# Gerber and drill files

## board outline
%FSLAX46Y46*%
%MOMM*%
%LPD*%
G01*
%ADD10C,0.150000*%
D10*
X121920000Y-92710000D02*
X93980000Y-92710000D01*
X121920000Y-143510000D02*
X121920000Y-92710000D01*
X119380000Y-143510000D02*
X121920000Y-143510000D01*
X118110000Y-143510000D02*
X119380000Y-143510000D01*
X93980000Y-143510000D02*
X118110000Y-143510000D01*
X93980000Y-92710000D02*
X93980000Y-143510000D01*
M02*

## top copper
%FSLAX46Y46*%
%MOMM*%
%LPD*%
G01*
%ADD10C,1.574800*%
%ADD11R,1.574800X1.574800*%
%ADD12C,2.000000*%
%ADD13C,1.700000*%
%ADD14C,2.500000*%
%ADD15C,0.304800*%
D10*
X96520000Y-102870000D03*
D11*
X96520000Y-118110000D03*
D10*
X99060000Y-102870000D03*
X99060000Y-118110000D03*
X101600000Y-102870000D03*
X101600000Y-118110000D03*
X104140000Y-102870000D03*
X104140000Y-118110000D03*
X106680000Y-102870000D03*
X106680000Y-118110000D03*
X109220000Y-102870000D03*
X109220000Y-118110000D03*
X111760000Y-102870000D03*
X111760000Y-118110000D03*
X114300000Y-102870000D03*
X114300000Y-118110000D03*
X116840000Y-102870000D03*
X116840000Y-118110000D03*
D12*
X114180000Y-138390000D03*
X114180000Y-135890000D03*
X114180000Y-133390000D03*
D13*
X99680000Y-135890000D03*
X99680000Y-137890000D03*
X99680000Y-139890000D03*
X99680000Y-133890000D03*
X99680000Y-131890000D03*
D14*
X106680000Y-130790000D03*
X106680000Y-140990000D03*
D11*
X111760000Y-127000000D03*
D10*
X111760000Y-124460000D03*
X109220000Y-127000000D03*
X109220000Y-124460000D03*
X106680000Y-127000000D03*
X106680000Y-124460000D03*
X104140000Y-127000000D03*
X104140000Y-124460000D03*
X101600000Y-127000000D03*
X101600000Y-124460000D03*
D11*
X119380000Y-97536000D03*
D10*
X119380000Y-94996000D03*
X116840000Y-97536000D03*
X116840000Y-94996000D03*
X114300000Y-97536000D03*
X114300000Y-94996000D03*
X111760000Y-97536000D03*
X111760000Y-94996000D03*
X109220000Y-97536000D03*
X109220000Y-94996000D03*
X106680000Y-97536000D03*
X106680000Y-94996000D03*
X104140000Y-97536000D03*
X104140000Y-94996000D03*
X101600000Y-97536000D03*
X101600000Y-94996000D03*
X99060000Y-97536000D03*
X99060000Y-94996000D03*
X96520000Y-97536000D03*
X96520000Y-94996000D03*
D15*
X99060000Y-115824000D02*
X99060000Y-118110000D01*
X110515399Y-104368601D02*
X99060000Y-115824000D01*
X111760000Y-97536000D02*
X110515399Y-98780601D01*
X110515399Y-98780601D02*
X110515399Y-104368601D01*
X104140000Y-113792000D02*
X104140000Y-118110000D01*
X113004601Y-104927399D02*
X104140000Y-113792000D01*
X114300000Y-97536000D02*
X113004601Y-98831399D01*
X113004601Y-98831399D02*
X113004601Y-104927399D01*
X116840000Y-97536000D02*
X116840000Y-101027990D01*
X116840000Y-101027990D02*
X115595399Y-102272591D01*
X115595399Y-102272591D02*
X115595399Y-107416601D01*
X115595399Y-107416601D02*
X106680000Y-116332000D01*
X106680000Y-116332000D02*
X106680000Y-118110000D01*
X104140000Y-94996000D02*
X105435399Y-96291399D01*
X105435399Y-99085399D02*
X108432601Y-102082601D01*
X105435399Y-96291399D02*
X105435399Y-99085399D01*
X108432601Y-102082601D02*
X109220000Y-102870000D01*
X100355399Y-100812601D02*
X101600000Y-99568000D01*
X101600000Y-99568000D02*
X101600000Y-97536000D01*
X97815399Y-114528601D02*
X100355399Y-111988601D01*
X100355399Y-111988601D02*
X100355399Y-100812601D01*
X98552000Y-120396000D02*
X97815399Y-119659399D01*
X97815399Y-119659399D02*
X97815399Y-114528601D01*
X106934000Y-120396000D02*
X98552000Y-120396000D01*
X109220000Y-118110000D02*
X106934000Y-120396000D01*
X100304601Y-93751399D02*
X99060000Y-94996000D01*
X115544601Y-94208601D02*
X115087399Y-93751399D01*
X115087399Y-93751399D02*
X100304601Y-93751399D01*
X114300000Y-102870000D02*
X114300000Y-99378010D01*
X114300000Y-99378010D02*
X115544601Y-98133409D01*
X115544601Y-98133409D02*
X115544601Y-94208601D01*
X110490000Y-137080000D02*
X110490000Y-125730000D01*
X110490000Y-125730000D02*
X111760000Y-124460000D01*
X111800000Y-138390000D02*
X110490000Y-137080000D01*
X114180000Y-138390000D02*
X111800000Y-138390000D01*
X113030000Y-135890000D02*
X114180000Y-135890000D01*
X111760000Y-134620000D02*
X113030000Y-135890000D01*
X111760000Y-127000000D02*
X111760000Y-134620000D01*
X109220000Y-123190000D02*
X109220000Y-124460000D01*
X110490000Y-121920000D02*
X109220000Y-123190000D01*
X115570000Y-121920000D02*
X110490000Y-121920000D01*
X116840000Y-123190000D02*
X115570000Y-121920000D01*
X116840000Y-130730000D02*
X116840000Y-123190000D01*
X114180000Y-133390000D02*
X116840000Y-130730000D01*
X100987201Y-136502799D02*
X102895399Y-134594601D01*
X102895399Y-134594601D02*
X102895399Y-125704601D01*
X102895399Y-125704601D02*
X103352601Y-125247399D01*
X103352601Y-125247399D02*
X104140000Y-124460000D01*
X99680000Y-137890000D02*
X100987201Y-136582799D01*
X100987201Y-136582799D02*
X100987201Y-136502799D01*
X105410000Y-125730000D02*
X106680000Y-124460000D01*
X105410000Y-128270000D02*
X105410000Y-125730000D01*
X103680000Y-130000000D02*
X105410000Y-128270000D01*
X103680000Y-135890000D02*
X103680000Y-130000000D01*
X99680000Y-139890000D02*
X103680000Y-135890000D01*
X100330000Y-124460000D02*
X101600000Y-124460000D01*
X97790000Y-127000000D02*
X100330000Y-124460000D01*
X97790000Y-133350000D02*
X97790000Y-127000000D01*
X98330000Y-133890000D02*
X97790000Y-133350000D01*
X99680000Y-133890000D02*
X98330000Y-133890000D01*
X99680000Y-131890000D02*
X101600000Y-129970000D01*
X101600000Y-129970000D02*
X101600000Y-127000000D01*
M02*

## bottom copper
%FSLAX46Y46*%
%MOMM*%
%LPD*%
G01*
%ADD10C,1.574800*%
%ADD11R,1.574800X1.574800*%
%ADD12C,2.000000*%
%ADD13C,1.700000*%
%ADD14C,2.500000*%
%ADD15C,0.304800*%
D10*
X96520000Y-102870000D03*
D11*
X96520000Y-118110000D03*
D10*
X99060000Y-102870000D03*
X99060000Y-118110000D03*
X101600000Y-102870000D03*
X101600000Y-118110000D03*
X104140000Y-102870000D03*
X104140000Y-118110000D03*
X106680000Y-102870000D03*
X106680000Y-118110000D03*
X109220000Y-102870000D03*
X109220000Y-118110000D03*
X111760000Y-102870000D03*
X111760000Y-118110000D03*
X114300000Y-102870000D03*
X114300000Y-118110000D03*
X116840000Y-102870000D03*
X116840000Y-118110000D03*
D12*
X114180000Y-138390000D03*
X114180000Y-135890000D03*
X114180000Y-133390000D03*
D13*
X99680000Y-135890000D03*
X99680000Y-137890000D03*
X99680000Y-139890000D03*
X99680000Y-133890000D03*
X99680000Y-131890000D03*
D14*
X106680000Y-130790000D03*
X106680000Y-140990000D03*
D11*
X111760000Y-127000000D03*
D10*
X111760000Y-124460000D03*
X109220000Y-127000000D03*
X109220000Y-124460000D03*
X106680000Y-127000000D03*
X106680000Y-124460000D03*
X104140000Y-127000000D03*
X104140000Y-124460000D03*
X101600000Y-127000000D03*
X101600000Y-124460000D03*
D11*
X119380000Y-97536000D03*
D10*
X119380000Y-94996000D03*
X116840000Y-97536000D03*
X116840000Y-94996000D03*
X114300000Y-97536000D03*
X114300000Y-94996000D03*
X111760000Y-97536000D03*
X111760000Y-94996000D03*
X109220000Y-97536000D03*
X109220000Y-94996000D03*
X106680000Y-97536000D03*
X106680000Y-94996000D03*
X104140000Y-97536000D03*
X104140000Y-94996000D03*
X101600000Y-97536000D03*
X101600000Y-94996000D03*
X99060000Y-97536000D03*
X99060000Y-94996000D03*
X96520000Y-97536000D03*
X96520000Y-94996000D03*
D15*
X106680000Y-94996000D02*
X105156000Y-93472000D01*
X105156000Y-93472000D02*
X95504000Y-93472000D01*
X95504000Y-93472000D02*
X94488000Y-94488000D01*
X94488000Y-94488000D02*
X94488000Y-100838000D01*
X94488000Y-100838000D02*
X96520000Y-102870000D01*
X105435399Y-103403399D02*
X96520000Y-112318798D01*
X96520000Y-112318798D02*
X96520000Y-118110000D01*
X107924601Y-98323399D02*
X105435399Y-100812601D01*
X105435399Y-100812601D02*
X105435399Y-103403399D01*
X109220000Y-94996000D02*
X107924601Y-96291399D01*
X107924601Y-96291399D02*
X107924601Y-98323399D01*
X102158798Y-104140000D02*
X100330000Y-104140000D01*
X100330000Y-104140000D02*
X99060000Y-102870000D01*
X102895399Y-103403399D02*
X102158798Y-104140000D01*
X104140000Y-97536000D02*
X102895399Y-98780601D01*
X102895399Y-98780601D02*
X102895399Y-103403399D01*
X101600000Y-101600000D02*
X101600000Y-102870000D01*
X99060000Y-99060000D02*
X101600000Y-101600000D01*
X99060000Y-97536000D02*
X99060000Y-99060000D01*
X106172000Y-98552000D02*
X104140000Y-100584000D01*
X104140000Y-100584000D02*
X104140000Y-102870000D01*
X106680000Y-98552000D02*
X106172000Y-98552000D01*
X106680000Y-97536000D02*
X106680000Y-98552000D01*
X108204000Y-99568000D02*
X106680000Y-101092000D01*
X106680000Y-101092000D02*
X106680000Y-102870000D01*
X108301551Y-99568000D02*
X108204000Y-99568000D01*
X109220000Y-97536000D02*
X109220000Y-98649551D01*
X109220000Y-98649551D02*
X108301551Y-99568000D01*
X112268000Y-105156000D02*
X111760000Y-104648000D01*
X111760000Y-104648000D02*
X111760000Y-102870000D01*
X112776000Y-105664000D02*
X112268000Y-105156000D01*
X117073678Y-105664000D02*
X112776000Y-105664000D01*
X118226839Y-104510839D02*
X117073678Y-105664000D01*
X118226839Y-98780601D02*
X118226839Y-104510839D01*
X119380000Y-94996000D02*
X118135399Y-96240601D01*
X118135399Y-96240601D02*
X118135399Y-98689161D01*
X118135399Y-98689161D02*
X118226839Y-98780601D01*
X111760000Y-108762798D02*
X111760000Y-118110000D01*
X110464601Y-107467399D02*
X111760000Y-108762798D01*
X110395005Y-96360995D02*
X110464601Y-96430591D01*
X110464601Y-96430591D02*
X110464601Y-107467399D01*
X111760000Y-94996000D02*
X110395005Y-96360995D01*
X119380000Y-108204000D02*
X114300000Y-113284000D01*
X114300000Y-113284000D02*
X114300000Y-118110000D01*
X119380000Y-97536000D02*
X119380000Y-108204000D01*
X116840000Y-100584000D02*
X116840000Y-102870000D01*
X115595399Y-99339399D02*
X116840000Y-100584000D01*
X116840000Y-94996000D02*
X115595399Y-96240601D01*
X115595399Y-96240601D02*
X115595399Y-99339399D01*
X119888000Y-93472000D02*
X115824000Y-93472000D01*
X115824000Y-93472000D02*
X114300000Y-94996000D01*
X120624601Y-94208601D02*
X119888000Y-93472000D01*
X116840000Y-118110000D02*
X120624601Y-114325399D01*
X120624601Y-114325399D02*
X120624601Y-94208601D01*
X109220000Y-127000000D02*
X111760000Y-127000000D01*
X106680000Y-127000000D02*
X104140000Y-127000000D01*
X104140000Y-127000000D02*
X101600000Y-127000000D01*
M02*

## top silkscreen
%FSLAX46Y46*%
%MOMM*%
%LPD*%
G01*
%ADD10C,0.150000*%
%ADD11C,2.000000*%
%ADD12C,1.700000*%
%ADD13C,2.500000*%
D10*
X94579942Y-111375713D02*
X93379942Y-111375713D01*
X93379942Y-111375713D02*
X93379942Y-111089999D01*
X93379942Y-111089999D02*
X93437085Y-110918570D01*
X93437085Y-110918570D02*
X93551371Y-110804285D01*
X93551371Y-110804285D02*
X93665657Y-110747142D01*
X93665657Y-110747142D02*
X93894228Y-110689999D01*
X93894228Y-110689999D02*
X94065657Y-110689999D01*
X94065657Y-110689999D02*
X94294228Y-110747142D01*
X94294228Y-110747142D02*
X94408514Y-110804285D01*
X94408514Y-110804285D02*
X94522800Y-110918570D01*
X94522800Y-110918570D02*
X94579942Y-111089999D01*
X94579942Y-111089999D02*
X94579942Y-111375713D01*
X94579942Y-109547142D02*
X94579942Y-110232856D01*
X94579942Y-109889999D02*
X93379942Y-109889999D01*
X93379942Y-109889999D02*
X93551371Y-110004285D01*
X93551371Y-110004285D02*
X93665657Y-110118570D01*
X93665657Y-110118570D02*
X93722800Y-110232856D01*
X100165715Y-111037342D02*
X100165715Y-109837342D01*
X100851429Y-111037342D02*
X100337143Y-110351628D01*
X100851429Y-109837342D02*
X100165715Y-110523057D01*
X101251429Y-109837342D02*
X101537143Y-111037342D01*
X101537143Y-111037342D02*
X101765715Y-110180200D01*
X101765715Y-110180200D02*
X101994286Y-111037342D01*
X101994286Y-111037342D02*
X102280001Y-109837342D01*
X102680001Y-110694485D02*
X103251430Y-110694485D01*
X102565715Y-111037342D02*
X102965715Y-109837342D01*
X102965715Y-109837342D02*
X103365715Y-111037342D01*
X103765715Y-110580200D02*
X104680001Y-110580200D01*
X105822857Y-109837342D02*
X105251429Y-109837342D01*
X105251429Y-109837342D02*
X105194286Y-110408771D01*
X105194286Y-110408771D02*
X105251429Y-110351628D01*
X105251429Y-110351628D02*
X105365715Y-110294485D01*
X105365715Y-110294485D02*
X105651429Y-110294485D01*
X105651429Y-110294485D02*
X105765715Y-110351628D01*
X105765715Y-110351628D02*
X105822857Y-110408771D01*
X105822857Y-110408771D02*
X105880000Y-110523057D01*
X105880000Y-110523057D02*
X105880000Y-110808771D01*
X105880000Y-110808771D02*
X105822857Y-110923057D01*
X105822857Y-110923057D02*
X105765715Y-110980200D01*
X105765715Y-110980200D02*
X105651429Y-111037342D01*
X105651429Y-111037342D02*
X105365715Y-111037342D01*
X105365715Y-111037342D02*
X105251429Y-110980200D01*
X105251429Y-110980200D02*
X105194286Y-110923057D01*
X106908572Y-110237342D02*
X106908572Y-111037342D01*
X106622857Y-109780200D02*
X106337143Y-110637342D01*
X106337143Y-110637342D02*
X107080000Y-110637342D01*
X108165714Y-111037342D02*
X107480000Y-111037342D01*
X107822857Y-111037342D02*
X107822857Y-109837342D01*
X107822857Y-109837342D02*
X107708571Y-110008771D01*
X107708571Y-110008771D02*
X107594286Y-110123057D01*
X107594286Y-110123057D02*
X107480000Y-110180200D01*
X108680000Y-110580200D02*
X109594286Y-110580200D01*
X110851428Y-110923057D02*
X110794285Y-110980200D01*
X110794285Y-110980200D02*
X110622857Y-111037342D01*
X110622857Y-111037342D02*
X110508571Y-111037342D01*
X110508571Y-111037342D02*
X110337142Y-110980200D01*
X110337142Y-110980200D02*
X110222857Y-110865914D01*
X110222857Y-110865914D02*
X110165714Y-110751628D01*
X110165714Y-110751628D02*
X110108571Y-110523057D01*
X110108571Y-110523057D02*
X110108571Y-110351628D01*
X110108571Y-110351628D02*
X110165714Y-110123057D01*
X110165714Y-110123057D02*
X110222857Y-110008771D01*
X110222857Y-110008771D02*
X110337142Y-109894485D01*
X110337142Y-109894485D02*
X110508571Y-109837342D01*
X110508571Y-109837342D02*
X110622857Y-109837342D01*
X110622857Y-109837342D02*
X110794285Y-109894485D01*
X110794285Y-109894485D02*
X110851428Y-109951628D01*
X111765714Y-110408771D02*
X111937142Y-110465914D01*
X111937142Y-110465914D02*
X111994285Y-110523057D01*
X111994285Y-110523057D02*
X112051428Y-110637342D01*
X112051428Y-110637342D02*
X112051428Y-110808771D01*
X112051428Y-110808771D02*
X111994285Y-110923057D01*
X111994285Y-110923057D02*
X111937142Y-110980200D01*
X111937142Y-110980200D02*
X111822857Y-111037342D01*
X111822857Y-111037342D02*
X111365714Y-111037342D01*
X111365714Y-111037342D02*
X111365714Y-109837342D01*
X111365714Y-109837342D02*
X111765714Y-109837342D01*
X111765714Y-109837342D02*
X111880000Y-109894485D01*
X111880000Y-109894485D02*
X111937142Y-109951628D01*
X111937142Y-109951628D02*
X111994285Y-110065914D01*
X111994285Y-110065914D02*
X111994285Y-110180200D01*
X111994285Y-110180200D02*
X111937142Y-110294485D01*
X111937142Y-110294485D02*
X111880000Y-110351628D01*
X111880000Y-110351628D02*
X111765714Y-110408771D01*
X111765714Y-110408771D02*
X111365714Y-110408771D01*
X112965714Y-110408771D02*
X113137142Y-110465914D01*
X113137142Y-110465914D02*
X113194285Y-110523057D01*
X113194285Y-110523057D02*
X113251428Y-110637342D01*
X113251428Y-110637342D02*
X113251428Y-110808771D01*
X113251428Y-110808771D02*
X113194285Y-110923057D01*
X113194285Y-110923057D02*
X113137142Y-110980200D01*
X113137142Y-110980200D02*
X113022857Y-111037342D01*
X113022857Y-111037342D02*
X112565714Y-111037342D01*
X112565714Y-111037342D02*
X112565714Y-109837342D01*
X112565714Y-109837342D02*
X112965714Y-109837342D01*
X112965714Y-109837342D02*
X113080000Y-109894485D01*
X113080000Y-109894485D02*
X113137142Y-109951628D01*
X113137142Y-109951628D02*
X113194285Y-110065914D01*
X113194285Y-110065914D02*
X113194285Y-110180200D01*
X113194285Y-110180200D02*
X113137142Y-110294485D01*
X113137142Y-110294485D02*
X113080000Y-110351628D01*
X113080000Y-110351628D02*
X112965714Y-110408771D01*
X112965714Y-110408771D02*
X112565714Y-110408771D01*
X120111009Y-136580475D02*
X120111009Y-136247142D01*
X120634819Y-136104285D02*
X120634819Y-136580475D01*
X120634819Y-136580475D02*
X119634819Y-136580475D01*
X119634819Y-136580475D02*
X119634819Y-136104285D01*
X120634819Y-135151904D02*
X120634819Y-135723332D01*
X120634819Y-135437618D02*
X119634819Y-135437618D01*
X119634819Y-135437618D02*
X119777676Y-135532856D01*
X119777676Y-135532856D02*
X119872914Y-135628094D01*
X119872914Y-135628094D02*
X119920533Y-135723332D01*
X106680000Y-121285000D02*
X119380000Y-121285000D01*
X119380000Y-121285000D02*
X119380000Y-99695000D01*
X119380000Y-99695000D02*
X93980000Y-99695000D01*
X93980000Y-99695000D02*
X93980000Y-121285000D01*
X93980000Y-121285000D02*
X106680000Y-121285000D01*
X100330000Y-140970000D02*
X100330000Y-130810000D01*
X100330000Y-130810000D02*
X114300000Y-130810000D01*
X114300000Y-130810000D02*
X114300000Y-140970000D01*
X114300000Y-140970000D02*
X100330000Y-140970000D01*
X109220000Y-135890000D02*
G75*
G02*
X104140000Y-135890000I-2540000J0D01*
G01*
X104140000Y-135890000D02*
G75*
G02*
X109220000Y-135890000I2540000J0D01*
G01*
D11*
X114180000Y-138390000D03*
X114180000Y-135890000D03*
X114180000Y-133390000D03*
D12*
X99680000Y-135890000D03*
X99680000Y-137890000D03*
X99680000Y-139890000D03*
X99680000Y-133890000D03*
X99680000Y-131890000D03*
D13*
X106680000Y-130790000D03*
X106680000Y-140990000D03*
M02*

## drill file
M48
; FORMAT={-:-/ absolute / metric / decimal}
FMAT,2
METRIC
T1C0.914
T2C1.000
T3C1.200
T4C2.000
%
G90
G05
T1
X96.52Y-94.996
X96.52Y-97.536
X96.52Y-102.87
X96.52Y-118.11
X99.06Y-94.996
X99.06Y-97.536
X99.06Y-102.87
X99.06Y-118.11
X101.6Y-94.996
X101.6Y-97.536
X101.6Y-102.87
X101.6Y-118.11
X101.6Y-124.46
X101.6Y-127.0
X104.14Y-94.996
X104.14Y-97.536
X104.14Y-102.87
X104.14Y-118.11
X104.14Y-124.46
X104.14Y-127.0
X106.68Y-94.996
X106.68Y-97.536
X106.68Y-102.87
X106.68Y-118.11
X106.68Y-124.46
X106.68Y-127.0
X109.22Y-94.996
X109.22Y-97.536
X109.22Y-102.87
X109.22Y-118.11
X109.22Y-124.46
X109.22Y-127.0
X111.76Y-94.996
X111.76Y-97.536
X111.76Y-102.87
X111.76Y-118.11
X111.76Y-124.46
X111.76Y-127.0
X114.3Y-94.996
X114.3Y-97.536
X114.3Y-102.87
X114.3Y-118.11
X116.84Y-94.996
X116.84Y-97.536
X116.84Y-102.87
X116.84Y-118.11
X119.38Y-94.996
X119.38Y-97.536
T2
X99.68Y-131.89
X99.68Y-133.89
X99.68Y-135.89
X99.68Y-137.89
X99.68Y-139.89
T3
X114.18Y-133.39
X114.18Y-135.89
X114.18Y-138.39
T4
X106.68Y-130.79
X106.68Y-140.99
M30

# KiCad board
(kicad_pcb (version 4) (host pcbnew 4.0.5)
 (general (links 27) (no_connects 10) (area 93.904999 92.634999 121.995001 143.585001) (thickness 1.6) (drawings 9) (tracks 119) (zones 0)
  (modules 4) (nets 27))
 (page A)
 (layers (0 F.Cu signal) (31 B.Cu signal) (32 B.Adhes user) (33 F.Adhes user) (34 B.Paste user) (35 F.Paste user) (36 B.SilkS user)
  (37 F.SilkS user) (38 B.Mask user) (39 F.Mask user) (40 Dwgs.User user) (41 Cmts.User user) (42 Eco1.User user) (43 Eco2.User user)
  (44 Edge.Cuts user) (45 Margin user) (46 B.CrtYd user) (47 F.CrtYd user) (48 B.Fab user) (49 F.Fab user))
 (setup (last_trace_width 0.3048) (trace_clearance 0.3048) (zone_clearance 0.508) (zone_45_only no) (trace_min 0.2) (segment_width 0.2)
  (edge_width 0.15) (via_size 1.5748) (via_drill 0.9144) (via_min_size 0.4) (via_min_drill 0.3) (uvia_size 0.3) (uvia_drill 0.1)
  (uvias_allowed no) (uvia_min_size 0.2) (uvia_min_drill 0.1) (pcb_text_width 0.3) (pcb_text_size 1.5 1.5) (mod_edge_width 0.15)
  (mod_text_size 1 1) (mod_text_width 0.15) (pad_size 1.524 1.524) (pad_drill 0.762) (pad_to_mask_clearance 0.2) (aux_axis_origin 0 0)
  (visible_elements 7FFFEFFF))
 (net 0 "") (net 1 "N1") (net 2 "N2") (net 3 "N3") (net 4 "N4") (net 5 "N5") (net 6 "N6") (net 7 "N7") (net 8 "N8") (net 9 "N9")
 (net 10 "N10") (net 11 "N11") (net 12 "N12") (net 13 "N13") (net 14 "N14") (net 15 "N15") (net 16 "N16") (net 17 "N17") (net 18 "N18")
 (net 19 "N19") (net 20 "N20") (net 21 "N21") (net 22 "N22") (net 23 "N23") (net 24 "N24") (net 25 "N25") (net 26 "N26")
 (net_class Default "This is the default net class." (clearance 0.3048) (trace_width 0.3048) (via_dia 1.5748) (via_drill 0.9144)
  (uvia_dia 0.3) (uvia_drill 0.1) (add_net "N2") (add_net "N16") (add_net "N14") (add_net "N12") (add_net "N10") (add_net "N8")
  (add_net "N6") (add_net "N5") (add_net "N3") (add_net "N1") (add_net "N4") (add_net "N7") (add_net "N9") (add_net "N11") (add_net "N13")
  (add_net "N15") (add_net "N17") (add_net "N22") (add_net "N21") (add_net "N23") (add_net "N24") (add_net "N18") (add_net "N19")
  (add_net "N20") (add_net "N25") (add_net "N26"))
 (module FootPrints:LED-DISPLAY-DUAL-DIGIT (layer F.Cu) (at 106.68 110.49)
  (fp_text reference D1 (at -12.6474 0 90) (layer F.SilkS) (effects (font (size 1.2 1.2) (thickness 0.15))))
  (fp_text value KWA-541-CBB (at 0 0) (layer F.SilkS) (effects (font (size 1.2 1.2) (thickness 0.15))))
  (fp_line (start 0 10.795) (end 12.7 10.795) (layer F.SilkS) (width 0.15))
  (fp_line (start 12.7 10.795) (end 12.7 -10.795) (layer F.SilkS) (width 0.15))
  (fp_line (start 12.7 -10.795) (end -12.7 -10.795) (layer F.SilkS) (width 0.15))
  (fp_line (start -12.7 -10.795) (end -12.7 10.795) (layer F.SilkS) (width 0.15))
  (fp_line (start -12.7 10.795) (end 0 10.795) (layer F.SilkS) (width 0.15))
  (pad 18 thru_hole circle (at -10.16 -7.62) (size 1.5748 1.5748) (drill 0.9144) (layers *.Cu *.Mask) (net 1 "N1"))
  (pad 1 thru_hole rect (at -10.16 7.62) (size 1.5748 1.5748) (drill 0.9144) (layers *.Cu *.Mask) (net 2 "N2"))
  (pad 17 thru_hole circle (at -7.62 -7.62) (size 1.5748 1.5748) (drill 0.9144) (layers *.Cu *.Mask) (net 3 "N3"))
  (pad 2 thru_hole circle (at -7.62 7.62) (size 1.5748 1.5748) (drill 0.9144) (layers *.Cu *.Mask) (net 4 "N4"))
  (pad 16 thru_hole circle (at -5.08 -7.62) (size 1.5748 1.5748) (drill 0.9144) (layers *.Cu *.Mask) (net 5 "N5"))
  (pad 3 thru_hole circle (at -5.08 7.62) (size 1.5748 1.5748) (drill 0.9144) (layers *.Cu *.Mask))
  (pad 15 thru_hole circle (at -2.54 -7.62) (size 1.5748 1.5748) (drill 0.9144) (layers *.Cu *.Mask) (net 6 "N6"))
  (pad 4 thru_hole circle (at -2.54 7.62) (size 1.5748 1.5748) (drill 0.9144) (layers *.Cu *.Mask) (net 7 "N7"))
  (pad 14 thru_hole circle (at 0 -7.62) (size 1.5748 1.5748) (drill 0.9144) (layers *.Cu *.Mask) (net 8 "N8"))
  (pad 5 thru_hole circle (at 0 7.62) (size 1.5748 1.5748) (drill 0.9144) (layers *.Cu *.Mask) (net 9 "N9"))
  (pad 13 thru_hole circle (at 2.54 -7.62) (size 1.5748 1.5748) (drill 0.9144) (layers *.Cu *.Mask) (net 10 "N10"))
  (pad 6 thru_hole circle (at 2.54 7.62) (size 1.5748 1.5748) (drill 0.9144) (layers *.Cu *.Mask) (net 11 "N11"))
  (pad 12 thru_hole circle (at 5.08 -7.62) (size 1.5748 1.5748) (drill 0.9144) (layers *.Cu *.Mask) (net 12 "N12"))
  (pad 7 thru_hole circle (at 5.08 7.62) (size 1.5748 1.5748) (drill 0.9144) (layers *.Cu *.Mask) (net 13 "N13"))
  (pad 11 thru_hole circle (at 7.62 -7.62) (size 1.5748 1.5748) (drill 0.9144) (layers *.Cu *.Mask) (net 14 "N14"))
  (pad 8 thru_hole circle (at 7.62 7.62) (size 1.5748 1.5748) (drill 0.9144) (layers *.Cu *.Mask) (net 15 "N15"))
  (pad 10 thru_hole circle (at 10.16 -7.62) (size 1.5748 1.5748) (drill 0.9144) (layers *.Cu *.Mask) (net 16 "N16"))
  (pad 9 thru_hole circle (at 10.16 7.62) (size 1.5748 1.5748) (drill 0.9144) (layers *.Cu *.Mask) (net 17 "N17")))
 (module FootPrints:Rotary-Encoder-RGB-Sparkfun (layer F.Cu) (at 106.68 135.89 90)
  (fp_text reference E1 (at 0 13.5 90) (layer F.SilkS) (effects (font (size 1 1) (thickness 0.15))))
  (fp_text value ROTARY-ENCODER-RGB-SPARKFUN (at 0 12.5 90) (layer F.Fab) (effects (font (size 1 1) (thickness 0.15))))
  (fp_line (start -5.08 -6.35) (end 5.08 -6.35) (layer F.SilkS) (width 0.15))
  (fp_line (start 5.08 -6.35) (end 5.08 7.62) (layer F.SilkS) (width 0.15))
  (fp_line (start 5.08 7.62) (end -5.08 7.62) (layer F.SilkS) (width 0.15))
  (fp_line (start -5.08 7.62) (end -5.08 -6.35) (layer F.SilkS) (width 0.15))
  (fp_circle (center 0 0) (end 2.54 0) (layer F.SilkS) (width 0.15))
  (pad 6 thru_hole circle (at -2.5 7.5 90) (size 2 2) (drill 1.2) (layers *.Cu *.Mask F.SilkS) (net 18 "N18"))
  (pad 7 thru_hole circle (at 0 7.5 90) (size 2 2) (drill 1.2) (layers *.Cu *.Mask F.SilkS) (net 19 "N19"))
  (pad 8 thru_hole circle (at 2.5 7.5 90) (size 2 2) (drill 1.2) (layers *.Cu *.Mask F.SilkS) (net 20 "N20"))
  (pad 3 thru_hole circle (at 0 -7 90) (size 1.7 1.7) (drill 1) (layers *.Cu *.Mask F.SilkS))
  (pad 2 thru_hole circle (at -2 -7 90) (size 1.7 1.7) (drill 1) (layers *.Cu *.Mask F.SilkS) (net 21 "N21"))
  (pad 1 thru_hole circle (at -4 -7 90) (size 1.7 1.7) (drill 1) (layers *.Cu *.Mask F.SilkS) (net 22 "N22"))
  (pad 4 thru_hole circle (at 2 -7 90) (size 1.7 1.7) (drill 1) (layers *.Cu *.Mask F.SilkS) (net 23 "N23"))
  (pad 5 thru_hole circle (at 4 -7 90) (size 1.7 1.7) (drill 1) (layers *.Cu *.Mask F.SilkS) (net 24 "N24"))
  (pad "" thru_hole circle (at 5.1 0 90) (size 2.5 2.5) (drill 2) (layers *.Cu *.Mask F.SilkS))
  (pad "" thru_hole circle (at -5.1 0 90) (size 2.5 2.5) (drill 2) (layers *.Cu *.Mask F.SilkS)))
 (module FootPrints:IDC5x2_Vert (layer B.Cu) (at 106.68 125.73)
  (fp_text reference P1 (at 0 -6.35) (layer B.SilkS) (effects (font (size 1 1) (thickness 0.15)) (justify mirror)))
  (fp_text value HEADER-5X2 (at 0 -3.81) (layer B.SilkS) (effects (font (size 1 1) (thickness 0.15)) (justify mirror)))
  (pad 1 thru_hole rect (at 5.08 1.27) (size 1.5748 1.5748) (drill 0.9144) (layers *.Cu *.Mask B.SilkS) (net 19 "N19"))
  (pad 2 thru_hole circle (at 5.08 -1.27) (size 1.5748 1.5748) (drill 0.9144) (layers *.Cu *.Mask B.SilkS) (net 18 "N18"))
  (pad 3 thru_hole circle (at 2.54 1.27) (size 1.5748 1.5748) (drill 0.9144) (layers *.Cu *.Mask B.SilkS) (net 19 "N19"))
  (pad 4 thru_hole circle (at 2.54 -1.27) (size 1.5748 1.5748) (drill 0.9144) (layers *.Cu *.Mask B.SilkS) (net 20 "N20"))
  (pad 5 thru_hole circle (at 0 1.27) (size 1.5748 1.5748) (drill 0.9144) (layers *.Cu *.Mask B.SilkS) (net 24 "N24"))
  (pad 6 thru_hole circle (at 0 -1.27) (size 1.5748 1.5748) (drill 0.9144) (layers *.Cu *.Mask B.SilkS) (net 22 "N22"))
  (pad 7 thru_hole circle (at -2.54 1.27) (size 1.5748 1.5748) (drill 0.9144) (layers *.Cu *.Mask B.SilkS) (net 24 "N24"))
  (pad 8 thru_hole circle (at -2.54 -1.27) (size 1.5748 1.5748) (drill 0.9144) (layers *.Cu *.Mask B.SilkS) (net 21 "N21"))
  (pad 9 thru_hole circle (at -5.08 1.27) (size 1.5748 1.5748) (drill 0.9144) (layers *.Cu *.Mask B.SilkS) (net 24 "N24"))
  (pad 10 thru_hole circle (at -5.08 -1.27) (size 1.5748 1.5748) (drill 0.9144) (layers *.Cu *.Mask B.SilkS) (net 23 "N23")))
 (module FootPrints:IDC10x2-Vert (layer B.Cu) (at 111.76 102.616 180)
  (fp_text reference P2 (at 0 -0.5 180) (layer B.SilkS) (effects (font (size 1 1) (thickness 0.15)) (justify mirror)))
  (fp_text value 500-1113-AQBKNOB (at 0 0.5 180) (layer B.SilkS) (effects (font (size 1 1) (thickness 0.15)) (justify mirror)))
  (pad 1 thru_hole rect (at -7.62 5.08 180) (size 1.5748 1.5748) (drill 0.9144) (layers *.Cu *.Mask) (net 15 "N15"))
  (pad 2 thru_hole circle (at -7.62 7.62 180) (size 1.5748 1.5748) (drill 0.9144) (layers *.Cu *.Mask) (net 12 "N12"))
  (pad 3 thru_hole circle (at -5.08 5.08 180) (size 1.5748 1.5748) (drill 0.9144) (layers *.Cu *.Mask) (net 9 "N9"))
  (pad 4 thru_hole circle (at -5.08 7.62 180) (size 1.5748 1.5748) (drill 0.9144) (layers *.Cu *.Mask) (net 16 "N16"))
  (pad 5 thru_hole circle (at -2.54 5.08 180) (size 1.5748 1.5748) (drill 0.9144) (layers *.Cu *.Mask) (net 7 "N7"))
  (pad 6 thru_hole circle (at -2.54 7.62 180) (size 1.5748 1.5748) (drill 0.9144) (layers *.Cu *.Mask) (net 17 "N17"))
  (pad 7 thru_hole circle (at 0 5.08 180) (size 1.5748 1.5748) (drill 0.9144) (layers *.Cu *.Mask) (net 4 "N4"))
  (pad 8 thru_hole circle (at 0 7.62 180) (size 1.5748 1.5748) (drill 0.9144) (layers *.Cu *.Mask) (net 13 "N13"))
  (pad 9 thru_hole circle (at 2.54 5.08 180) (size 1.5748 1.5748) (drill 0.9144) (layers *.Cu *.Mask) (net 8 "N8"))
  (pad 10 thru_hole circle (at 2.54 7.62 180) (size 1.5748 1.5748) (drill 0.9144) (layers *.Cu *.Mask) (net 2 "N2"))
  (pad 11 thru_hole circle (at 5.08 5.08 180) (size 1.5748 1.5748) (drill 0.9144) (layers *.Cu *.Mask) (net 6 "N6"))
  (pad 12 thru_hole circle (at 5.08 7.62 180) (size 1.5748 1.5748) (drill 0.9144) (layers *.Cu *.Mask) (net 1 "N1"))
  (pad 13 thru_hole circle (at 7.62 5.08 180) (size 1.5748 1.5748) (drill 0.9144) (layers *.Cu *.Mask) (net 3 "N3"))
  (pad 14 thru_hole circle (at 7.62 7.62 180) (size 1.5748 1.5748) (drill 0.9144) (layers *.Cu *.Mask) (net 10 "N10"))
  (pad 15 thru_hole circle (at 10.16 5.08 180) (size 1.5748 1.5748) (drill 0.9144) (layers *.Cu *.Mask) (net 11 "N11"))
  (pad 16 thru_hole circle (at 10.16 7.62 180) (size 1.5748 1.5748) (drill 0.9144) (layers *.Cu *.Mask))
  (pad 17 thru_hole circle (at 12.7 5.08 180) (size 1.5748 1.5748) (drill 0.9144) (layers *.Cu *.Mask) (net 5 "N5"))
  (pad 18 thru_hole circle (at 12.7 7.62 180) (size 1.5748 1.5748) (drill 0.9144) (layers *.Cu *.Mask) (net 14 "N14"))
  (pad 19 thru_hole circle (at 15.24 5.08 180) (size 1.5748 1.5748) (drill 0.9144) (layers *.Cu *.Mask) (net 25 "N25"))
  (pad 20 thru_hole circle (at 15.24 7.62 180) (size 1.5748 1.5748) (drill 0.9144) (layers *.Cu *.Mask) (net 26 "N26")))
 (gr_line (start 121.92 92.71) (end 93.98 92.71) (angle 90) (layer Edge.Cuts) (width 0.15))
 (gr_line (start 121.92 143.51) (end 121.92 92.71) (angle 90) (layer Edge.Cuts) (width 0.15))
 (gr_line (start 119.38 143.51) (end 121.92 143.51) (angle 90) (layer Edge.Cuts) (width 0.15))
 (gr_line (start 118.11 143.51) (end 119.38 143.51) (angle 90) (layer Edge.Cuts) (width 0.15))
 (gr_line (start 93.98 143.51) (end 118.11 143.51) (angle 90) (layer Edge.Cuts) (width 0.15))
 (gr_line (start 93.98 92.71) (end 93.98 143.51) (angle 90) (layer Edge.Cuts) (width 0.15))
 (segment (start 106.68 94.996) (end 105.156 93.472) (width 0.3048) (layer B.Cu) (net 1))
 (segment (start 105.156 93.472) (end 95.504 93.472) (width 0.3048) (layer B.Cu) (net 1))
 (segment (start 95.504 93.472) (end 94.488 94.488) (width 0.3048) (layer B.Cu) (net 1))
 (segment (start 94.488 94.488) (end 94.488 100.838) (width 0.3048) (layer B.Cu) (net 1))
 (segment (start 94.488 100.838) (end 96.52 102.87) (width 0.3048) (layer B.Cu) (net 1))
 (segment (start 105.435399 103.403399) (end 96.52 112.318798) (width 0.3048) (layer B.Cu) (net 2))
 (segment (start 96.52 112.318798) (end 96.52 118.11) (width 0.3048) (layer B.Cu) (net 2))
 (segment (start 107.924601 98.323399) (end 105.435399 100.812601) (width 0.3048) (layer B.Cu) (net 2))
 (segment (start 105.435399 100.812601) (end 105.435399 103.403399) (width 0.3048) (layer B.Cu) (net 2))
 (segment (start 109.22 94.996) (end 107.924601 96.291399) (width 0.3048) (layer B.Cu) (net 2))
 (segment (start 107.924601 96.291399) (end 107.924601 98.323399) (width 0.3048) (layer B.Cu) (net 2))
 (segment (start 102.158798 104.14) (end 100.33 104.14) (width 0.3048) (layer B.Cu) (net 3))
 (segment (start 100.33 104.14) (end 99.06 102.87) (width 0.3048) (layer B.Cu) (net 3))
 (segment (start 102.895399 103.403399) (end 102.158798 104.14) (width 0.3048) (layer B.Cu) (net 3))
 (segment (start 104.14 97.536) (end 102.895399 98.780601) (width 0.3048) (layer B.Cu) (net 3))
 (segment (start 102.895399 98.780601) (end 102.895399 103.403399) (width 0.3048) (layer B.Cu) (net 3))
 (segment (start 99.06 115.824) (end 99.06 118.11) (width 0.3048) (layer F.Cu) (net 4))
 (segment (start 110.515399 104.368601) (end 99.06 115.824) (width 0.3048) (layer F.Cu) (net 4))
 (segment (start 111.76 97.536) (end 110.515399 98.780601) (width 0.3048) (layer F.Cu) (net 4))
 (segment (start 110.515399 98.780601) (end 110.515399 104.368601) (width 0.3048) (layer F.Cu) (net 4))
 (segment (start 101.6 101.6) (end 101.6 102.87) (width 0.3048) (layer B.Cu) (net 5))
 (segment (start 99.06 99.06) (end 101.6 101.6) (width 0.3048) (layer B.Cu) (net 5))
 (segment (start 99.06 97.536) (end 99.06 99.06) (width 0.3048) (layer B.Cu) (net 5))
 (segment (start 106.172 98.552) (end 104.14 100.584) (width 0.3048) (layer B.Cu) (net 6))
 (segment (start 104.14 100.584) (end 104.14 102.87) (width 0.3048) (layer B.Cu) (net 6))
 (segment (start 106.68 98.552) (end 106.172 98.552) (width 0.3048) (layer B.Cu) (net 6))
 (segment (start 106.68 97.536) (end 106.68 98.552) (width 0.3048) (layer B.Cu) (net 6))
 (segment (start 104.14 113.792) (end 104.14 118.11) (width 0.3048) (layer F.Cu) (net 7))
 (segment (start 113.004601 104.927399) (end 104.14 113.792) (width 0.3048) (layer F.Cu) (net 7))
 (segment (start 114.3 97.536) (end 113.004601 98.831399) (width 0.3048) (layer F.Cu) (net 7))
 (segment (start 113.004601 98.831399) (end 113.004601 104.927399) (width 0.3048) (layer F.Cu) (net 7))
 (segment (start 108.204 99.568) (end 106.68 101.092) (width 0.3048) (layer B.Cu) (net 8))
 (segment (start 106.68 101.092) (end 106.68 102.87) (width 0.3048) (layer B.Cu) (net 8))
 (segment (start 108.301551 99.568) (end 108.204 99.568) (width 0.3048) (layer B.Cu) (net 8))
 (segment (start 109.22 97.536) (end 109.22 98.649551) (width 0.3048) (layer B.Cu) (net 8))
 (segment (start 109.22 98.649551) (end 108.301551 99.568) (width 0.3048) (layer B.Cu) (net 8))
 (segment (start 116.84 97.536) (end 116.84 101.02799) (width 0.3048) (layer F.Cu) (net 9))
 (segment (start 116.84 101.02799) (end 115.595399 102.272591) (width 0.3048) (layer F.Cu) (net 9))
 (segment (start 115.595399 102.272591) (end 115.595399 107.416601) (width 0.3048) (layer F.Cu) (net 9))
 (segment (start 115.595399 107.416601) (end 106.68 116.332) (width 0.3048) (layer F.Cu) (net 9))
 (segment (start 106.68 116.332) (end 106.68 118.11) (width 0.3048) (layer F.Cu) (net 9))
 (segment (start 104.14 94.996) (end 105.435399 96.291399) (width 0.3048) (layer F.Cu) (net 10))
 (segment (start 105.435399 99.085399) (end 108.432601 102.082601) (width 0.3048) (layer F.Cu) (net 10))
 (segment (start 105.435399 96.291399) (end 105.435399 99.085399) (width 0.3048) (layer F.Cu) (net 10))
 (segment (start 108.432601 102.082601) (end 109.22 102.87) (width 0.3048) (layer F.Cu) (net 10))
 (segment (start 100.355399 100.812601) (end 101.6 99.568) (width 0.3048) (layer F.Cu) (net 11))
 (segment (start 101.6 99.568) (end 101.6 97.536) (width 0.3048) (layer F.Cu) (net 11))
 (segment (start 97.815399 114.528601) (end 100.355399 111.988601) (width 0.3048) (layer F.Cu) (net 11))
 (segment (start 100.355399 111.988601) (end 100.355399 100.812601) (width 0.3048) (layer F.Cu) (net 11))
 (segment (start 98.552 120.396) (end 97.815399 119.659399) (width 0.3048) (layer F.Cu) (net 11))
 (segment (start 97.815399 119.659399) (end 97.815399 114.528601) (width 0.3048) (layer F.Cu) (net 11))
 (segment (start 106.934 120.396) (end 98.552 120.396) (width 0.3048) (layer F.Cu) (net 11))
 (segment (start 109.22 118.11) (end 106.934 120.396) (width 0.3048) (layer F.Cu) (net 11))
 (segment (start 112.268 105.156) (end 111.76 104.648) (width 0.3048) (layer B.Cu) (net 12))
 (segment (start 111.76 104.648) (end 111.76 102.87) (width 0.3048) (layer B.Cu) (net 12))
 (segment (start 112.776 105.664) (end 112.268 105.156) (width 0.3048) (layer B.Cu) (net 12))
 (segment (start 117.073678 105.664) (end 112.776 105.664) (width 0.3048) (layer B.Cu) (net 12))
 (segment (start 118.226839 104.510839) (end 117.073678 105.664) (width 0.3048) (layer B.Cu) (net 12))
 (segment (start 118.226839 98.780601) (end 118.226839 104.510839) (width 0.3048) (layer B.Cu) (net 12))
 (segment (start 119.38 94.996) (end 118.135399 96.240601) (width 0.3048) (layer B.Cu) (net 12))
 (segment (start 118.135399 96.240601) (end 118.135399 98.689161) (width 0.3048) (layer B.Cu) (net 12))
 (segment (start 118.135399 98.689161) (end 118.226839 98.780601) (width 0.3048) (layer B.Cu) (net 12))
 (segment (start 111.76 108.762798) (end 111.76 118.11) (width 0.3048) (layer B.Cu) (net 13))
 (segment (start 110.464601 107.467399) (end 111.76 108.762798) (width 0.3048) (layer B.Cu) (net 13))
 (segment (start 110.395005 96.360995) (end 110.464601 96.430591) (width 0.3048) (layer B.Cu) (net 13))
 (segment (start 110.464601 96.430591) (end 110.464601 107.467399) (width 0.3048) (layer B.Cu) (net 13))
 (segment (start 111.76 94.996) (end 110.395005 96.360995) (width 0.3048) (layer B.Cu) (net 13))
 (segment (start 100.304601 93.751399) (end 99.06 94.996) (width 0.3048) (layer F.Cu) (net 14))
 (segment (start 115.544601 94.208601) (end 115.087399 93.751399) (width 0.3048) (layer F.Cu) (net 14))
 (segment (start 115.087399 93.751399) (end 100.304601 93.751399) (width 0.3048) (layer F.Cu) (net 14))
 (segment (start 114.3 102.87) (end 114.3 99.37801) (width 0.3048) (layer F.Cu) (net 14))
 (segment (start 114.3 99.37801) (end 115.544601 98.133409) (width 0.3048) (layer F.Cu) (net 14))
 (segment (start 115.544601 98.133409) (end 115.544601 94.208601) (width 0.3048) (layer F.Cu) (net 14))
 (segment (start 119.38 108.204) (end 114.3 113.284) (width 0.3048) (layer B.Cu) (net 15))
 (segment (start 114.3 113.284) (end 114.3 118.11) (width 0.3048) (layer B.Cu) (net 15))
 (segment (start 119.38 97.536) (end 119.38 108.204) (width 0.3048) (layer B.Cu) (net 15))
 (segment (start 116.84 100.584) (end 116.84 102.87) (width 0.3048) (layer B.Cu) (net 16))
 (segment (start 115.595399 99.339399) (end 116.84 100.584) (width 0.3048) (layer B.Cu) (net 16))
 (segment (start 116.84 94.996) (end 115.595399 96.240601) (width 0.3048) (layer B.Cu) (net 16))
 (segment (start 115.595399 96.240601) (end 115.595399 99.339399) (width 0.3048) (layer B.Cu) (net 16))
 (segment (start 119.888 93.472) (end 115.824 93.472) (width 0.3048) (layer B.Cu) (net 17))
 (segment (start 115.824 93.472) (end 114.3 94.996) (width 0.3048) (layer B.Cu) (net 17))
 (segment (start 120.624601 94.208601) (end 119.888 93.472) (width 0.3048) (layer B.Cu) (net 17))
 (segment (start 116.84 118.11) (end 120.624601 114.325399) (width 0.3048) (layer B.Cu) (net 17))
 (segment (start 120.624601 114.325399) (end 120.624601 94.208601) (width 0.3048) (layer B.Cu) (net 17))
 (segment (start 110.49 137.08) (end 110.49 125.73) (width 0.3048) (layer F.Cu) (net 18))
 (segment (start 110.49 125.73) (end 111.76 124.46) (width 0.3048) (layer F.Cu) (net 18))
 (segment (start 111.8 138.39) (end 110.49 137.08) (width 0.3048) (layer F.Cu) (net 18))
 (segment (start 114.18 138.39) (end 111.8 138.39) (width 0.3048) (layer F.Cu) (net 18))
 (segment (start 109.22 127) (end 111.76 127) (width 0.3048) (layer B.Cu) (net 19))
 (segment (start 113.03 135.89) (end 114.18 135.89) (width 0.3048) (layer F.Cu) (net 19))
 (segment (start 111.76 134.62) (end 113.03 135.89) (width 0.3048) (layer F.Cu) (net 19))
 (segment (start 111.76 127) (end 111.76 134.62) (width 0.3048) (layer F.Cu) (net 19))
 (segment (start 109.22 123.19) (end 109.22 124.46) (width 0.3048) (layer F.Cu) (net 20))
 (segment (start 110.49 121.92) (end 109.22 123.19) (width 0.3048) (layer F.Cu) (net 20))
 (segment (start 115.57 121.92) (end 110.49 121.92) (width 0.3048) (layer F.Cu) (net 20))
 (segment (start 116.84 123.19) (end 115.57 121.92) (width 0.3048) (layer F.Cu) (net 20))
 (segment (start 116.84 130.73) (end 116.84 123.19) (width 0.3048) (layer F.Cu) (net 20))
 (segment (start 114.18 133.39) (end 116.84 130.73) (width 0.3048) (layer F.Cu) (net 20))
 (segment (start 100.987201 136.502799) (end 102.895399 134.594601) (width 0.3048) (layer F.Cu) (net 21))
 (segment (start 102.895399 134.594601) (end 102.895399 125.704601) (width 0.3048) (layer F.Cu) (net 21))
 (segment (start 102.895399 125.704601) (end 103.352601 125.247399) (width 0.3048) (layer F.Cu) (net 21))
 (segment (start 103.352601 125.247399) (end 104.14 124.46) (width 0.3048) (layer F.Cu) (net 21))
 (segment (start 99.68 137.89) (end 100.987201 136.582799) (width 0.3048) (layer F.Cu) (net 21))
 (segment (start 100.987201 136.582799) (end 100.987201 136.502799) (width 0.3048) (layer F.Cu) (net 21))
 (segment (start 105.41 125.73) (end 106.68 124.46) (width 0.3048) (layer F.Cu) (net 22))
 (segment (start 105.41 128.27) (end 105.41 125.73) (width 0.3048) (layer F.Cu) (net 22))
 (segment (start 103.68 130) (end 105.41 128.27) (width 0.3048) (layer F.Cu) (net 22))
 (segment (start 103.68 135.89) (end 103.68 130) (width 0.3048) (layer F.Cu) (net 22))
 (segment (start 99.68 139.89) (end 103.68 135.89) (width 0.3048) (layer F.Cu) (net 22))
 (segment (start 100.33 124.46) (end 101.6 124.46) (width 0.3048) (layer F.Cu) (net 23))
 (segment (start 97.79 127) (end 100.33 124.46) (width 0.3048) (layer F.Cu) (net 23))
 (segment (start 97.79 133.35) (end 97.79 127) (width 0.3048) (layer F.Cu) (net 23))
 (segment (start 98.33 133.89) (end 97.79 133.35) (width 0.3048) (layer F.Cu) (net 23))
 (segment (start 99.68 133.89) (end 98.33 133.89) (width 0.3048) (layer F.Cu) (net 23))
 (segment (start 106.68 127) (end 104.14 127) (width 0.3048) (layer B.Cu) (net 24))
 (segment (start 104.14 127) (end 101.6 127) (width 0.3048) (layer B.Cu) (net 24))
 (segment (start 99.68 131.89) (end 101.6 129.97) (width 0.3048) (layer F.Cu) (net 24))
 (segment (start 101.6 129.97) (end 101.6 127) (width 0.3048) (layer F.Cu) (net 24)))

